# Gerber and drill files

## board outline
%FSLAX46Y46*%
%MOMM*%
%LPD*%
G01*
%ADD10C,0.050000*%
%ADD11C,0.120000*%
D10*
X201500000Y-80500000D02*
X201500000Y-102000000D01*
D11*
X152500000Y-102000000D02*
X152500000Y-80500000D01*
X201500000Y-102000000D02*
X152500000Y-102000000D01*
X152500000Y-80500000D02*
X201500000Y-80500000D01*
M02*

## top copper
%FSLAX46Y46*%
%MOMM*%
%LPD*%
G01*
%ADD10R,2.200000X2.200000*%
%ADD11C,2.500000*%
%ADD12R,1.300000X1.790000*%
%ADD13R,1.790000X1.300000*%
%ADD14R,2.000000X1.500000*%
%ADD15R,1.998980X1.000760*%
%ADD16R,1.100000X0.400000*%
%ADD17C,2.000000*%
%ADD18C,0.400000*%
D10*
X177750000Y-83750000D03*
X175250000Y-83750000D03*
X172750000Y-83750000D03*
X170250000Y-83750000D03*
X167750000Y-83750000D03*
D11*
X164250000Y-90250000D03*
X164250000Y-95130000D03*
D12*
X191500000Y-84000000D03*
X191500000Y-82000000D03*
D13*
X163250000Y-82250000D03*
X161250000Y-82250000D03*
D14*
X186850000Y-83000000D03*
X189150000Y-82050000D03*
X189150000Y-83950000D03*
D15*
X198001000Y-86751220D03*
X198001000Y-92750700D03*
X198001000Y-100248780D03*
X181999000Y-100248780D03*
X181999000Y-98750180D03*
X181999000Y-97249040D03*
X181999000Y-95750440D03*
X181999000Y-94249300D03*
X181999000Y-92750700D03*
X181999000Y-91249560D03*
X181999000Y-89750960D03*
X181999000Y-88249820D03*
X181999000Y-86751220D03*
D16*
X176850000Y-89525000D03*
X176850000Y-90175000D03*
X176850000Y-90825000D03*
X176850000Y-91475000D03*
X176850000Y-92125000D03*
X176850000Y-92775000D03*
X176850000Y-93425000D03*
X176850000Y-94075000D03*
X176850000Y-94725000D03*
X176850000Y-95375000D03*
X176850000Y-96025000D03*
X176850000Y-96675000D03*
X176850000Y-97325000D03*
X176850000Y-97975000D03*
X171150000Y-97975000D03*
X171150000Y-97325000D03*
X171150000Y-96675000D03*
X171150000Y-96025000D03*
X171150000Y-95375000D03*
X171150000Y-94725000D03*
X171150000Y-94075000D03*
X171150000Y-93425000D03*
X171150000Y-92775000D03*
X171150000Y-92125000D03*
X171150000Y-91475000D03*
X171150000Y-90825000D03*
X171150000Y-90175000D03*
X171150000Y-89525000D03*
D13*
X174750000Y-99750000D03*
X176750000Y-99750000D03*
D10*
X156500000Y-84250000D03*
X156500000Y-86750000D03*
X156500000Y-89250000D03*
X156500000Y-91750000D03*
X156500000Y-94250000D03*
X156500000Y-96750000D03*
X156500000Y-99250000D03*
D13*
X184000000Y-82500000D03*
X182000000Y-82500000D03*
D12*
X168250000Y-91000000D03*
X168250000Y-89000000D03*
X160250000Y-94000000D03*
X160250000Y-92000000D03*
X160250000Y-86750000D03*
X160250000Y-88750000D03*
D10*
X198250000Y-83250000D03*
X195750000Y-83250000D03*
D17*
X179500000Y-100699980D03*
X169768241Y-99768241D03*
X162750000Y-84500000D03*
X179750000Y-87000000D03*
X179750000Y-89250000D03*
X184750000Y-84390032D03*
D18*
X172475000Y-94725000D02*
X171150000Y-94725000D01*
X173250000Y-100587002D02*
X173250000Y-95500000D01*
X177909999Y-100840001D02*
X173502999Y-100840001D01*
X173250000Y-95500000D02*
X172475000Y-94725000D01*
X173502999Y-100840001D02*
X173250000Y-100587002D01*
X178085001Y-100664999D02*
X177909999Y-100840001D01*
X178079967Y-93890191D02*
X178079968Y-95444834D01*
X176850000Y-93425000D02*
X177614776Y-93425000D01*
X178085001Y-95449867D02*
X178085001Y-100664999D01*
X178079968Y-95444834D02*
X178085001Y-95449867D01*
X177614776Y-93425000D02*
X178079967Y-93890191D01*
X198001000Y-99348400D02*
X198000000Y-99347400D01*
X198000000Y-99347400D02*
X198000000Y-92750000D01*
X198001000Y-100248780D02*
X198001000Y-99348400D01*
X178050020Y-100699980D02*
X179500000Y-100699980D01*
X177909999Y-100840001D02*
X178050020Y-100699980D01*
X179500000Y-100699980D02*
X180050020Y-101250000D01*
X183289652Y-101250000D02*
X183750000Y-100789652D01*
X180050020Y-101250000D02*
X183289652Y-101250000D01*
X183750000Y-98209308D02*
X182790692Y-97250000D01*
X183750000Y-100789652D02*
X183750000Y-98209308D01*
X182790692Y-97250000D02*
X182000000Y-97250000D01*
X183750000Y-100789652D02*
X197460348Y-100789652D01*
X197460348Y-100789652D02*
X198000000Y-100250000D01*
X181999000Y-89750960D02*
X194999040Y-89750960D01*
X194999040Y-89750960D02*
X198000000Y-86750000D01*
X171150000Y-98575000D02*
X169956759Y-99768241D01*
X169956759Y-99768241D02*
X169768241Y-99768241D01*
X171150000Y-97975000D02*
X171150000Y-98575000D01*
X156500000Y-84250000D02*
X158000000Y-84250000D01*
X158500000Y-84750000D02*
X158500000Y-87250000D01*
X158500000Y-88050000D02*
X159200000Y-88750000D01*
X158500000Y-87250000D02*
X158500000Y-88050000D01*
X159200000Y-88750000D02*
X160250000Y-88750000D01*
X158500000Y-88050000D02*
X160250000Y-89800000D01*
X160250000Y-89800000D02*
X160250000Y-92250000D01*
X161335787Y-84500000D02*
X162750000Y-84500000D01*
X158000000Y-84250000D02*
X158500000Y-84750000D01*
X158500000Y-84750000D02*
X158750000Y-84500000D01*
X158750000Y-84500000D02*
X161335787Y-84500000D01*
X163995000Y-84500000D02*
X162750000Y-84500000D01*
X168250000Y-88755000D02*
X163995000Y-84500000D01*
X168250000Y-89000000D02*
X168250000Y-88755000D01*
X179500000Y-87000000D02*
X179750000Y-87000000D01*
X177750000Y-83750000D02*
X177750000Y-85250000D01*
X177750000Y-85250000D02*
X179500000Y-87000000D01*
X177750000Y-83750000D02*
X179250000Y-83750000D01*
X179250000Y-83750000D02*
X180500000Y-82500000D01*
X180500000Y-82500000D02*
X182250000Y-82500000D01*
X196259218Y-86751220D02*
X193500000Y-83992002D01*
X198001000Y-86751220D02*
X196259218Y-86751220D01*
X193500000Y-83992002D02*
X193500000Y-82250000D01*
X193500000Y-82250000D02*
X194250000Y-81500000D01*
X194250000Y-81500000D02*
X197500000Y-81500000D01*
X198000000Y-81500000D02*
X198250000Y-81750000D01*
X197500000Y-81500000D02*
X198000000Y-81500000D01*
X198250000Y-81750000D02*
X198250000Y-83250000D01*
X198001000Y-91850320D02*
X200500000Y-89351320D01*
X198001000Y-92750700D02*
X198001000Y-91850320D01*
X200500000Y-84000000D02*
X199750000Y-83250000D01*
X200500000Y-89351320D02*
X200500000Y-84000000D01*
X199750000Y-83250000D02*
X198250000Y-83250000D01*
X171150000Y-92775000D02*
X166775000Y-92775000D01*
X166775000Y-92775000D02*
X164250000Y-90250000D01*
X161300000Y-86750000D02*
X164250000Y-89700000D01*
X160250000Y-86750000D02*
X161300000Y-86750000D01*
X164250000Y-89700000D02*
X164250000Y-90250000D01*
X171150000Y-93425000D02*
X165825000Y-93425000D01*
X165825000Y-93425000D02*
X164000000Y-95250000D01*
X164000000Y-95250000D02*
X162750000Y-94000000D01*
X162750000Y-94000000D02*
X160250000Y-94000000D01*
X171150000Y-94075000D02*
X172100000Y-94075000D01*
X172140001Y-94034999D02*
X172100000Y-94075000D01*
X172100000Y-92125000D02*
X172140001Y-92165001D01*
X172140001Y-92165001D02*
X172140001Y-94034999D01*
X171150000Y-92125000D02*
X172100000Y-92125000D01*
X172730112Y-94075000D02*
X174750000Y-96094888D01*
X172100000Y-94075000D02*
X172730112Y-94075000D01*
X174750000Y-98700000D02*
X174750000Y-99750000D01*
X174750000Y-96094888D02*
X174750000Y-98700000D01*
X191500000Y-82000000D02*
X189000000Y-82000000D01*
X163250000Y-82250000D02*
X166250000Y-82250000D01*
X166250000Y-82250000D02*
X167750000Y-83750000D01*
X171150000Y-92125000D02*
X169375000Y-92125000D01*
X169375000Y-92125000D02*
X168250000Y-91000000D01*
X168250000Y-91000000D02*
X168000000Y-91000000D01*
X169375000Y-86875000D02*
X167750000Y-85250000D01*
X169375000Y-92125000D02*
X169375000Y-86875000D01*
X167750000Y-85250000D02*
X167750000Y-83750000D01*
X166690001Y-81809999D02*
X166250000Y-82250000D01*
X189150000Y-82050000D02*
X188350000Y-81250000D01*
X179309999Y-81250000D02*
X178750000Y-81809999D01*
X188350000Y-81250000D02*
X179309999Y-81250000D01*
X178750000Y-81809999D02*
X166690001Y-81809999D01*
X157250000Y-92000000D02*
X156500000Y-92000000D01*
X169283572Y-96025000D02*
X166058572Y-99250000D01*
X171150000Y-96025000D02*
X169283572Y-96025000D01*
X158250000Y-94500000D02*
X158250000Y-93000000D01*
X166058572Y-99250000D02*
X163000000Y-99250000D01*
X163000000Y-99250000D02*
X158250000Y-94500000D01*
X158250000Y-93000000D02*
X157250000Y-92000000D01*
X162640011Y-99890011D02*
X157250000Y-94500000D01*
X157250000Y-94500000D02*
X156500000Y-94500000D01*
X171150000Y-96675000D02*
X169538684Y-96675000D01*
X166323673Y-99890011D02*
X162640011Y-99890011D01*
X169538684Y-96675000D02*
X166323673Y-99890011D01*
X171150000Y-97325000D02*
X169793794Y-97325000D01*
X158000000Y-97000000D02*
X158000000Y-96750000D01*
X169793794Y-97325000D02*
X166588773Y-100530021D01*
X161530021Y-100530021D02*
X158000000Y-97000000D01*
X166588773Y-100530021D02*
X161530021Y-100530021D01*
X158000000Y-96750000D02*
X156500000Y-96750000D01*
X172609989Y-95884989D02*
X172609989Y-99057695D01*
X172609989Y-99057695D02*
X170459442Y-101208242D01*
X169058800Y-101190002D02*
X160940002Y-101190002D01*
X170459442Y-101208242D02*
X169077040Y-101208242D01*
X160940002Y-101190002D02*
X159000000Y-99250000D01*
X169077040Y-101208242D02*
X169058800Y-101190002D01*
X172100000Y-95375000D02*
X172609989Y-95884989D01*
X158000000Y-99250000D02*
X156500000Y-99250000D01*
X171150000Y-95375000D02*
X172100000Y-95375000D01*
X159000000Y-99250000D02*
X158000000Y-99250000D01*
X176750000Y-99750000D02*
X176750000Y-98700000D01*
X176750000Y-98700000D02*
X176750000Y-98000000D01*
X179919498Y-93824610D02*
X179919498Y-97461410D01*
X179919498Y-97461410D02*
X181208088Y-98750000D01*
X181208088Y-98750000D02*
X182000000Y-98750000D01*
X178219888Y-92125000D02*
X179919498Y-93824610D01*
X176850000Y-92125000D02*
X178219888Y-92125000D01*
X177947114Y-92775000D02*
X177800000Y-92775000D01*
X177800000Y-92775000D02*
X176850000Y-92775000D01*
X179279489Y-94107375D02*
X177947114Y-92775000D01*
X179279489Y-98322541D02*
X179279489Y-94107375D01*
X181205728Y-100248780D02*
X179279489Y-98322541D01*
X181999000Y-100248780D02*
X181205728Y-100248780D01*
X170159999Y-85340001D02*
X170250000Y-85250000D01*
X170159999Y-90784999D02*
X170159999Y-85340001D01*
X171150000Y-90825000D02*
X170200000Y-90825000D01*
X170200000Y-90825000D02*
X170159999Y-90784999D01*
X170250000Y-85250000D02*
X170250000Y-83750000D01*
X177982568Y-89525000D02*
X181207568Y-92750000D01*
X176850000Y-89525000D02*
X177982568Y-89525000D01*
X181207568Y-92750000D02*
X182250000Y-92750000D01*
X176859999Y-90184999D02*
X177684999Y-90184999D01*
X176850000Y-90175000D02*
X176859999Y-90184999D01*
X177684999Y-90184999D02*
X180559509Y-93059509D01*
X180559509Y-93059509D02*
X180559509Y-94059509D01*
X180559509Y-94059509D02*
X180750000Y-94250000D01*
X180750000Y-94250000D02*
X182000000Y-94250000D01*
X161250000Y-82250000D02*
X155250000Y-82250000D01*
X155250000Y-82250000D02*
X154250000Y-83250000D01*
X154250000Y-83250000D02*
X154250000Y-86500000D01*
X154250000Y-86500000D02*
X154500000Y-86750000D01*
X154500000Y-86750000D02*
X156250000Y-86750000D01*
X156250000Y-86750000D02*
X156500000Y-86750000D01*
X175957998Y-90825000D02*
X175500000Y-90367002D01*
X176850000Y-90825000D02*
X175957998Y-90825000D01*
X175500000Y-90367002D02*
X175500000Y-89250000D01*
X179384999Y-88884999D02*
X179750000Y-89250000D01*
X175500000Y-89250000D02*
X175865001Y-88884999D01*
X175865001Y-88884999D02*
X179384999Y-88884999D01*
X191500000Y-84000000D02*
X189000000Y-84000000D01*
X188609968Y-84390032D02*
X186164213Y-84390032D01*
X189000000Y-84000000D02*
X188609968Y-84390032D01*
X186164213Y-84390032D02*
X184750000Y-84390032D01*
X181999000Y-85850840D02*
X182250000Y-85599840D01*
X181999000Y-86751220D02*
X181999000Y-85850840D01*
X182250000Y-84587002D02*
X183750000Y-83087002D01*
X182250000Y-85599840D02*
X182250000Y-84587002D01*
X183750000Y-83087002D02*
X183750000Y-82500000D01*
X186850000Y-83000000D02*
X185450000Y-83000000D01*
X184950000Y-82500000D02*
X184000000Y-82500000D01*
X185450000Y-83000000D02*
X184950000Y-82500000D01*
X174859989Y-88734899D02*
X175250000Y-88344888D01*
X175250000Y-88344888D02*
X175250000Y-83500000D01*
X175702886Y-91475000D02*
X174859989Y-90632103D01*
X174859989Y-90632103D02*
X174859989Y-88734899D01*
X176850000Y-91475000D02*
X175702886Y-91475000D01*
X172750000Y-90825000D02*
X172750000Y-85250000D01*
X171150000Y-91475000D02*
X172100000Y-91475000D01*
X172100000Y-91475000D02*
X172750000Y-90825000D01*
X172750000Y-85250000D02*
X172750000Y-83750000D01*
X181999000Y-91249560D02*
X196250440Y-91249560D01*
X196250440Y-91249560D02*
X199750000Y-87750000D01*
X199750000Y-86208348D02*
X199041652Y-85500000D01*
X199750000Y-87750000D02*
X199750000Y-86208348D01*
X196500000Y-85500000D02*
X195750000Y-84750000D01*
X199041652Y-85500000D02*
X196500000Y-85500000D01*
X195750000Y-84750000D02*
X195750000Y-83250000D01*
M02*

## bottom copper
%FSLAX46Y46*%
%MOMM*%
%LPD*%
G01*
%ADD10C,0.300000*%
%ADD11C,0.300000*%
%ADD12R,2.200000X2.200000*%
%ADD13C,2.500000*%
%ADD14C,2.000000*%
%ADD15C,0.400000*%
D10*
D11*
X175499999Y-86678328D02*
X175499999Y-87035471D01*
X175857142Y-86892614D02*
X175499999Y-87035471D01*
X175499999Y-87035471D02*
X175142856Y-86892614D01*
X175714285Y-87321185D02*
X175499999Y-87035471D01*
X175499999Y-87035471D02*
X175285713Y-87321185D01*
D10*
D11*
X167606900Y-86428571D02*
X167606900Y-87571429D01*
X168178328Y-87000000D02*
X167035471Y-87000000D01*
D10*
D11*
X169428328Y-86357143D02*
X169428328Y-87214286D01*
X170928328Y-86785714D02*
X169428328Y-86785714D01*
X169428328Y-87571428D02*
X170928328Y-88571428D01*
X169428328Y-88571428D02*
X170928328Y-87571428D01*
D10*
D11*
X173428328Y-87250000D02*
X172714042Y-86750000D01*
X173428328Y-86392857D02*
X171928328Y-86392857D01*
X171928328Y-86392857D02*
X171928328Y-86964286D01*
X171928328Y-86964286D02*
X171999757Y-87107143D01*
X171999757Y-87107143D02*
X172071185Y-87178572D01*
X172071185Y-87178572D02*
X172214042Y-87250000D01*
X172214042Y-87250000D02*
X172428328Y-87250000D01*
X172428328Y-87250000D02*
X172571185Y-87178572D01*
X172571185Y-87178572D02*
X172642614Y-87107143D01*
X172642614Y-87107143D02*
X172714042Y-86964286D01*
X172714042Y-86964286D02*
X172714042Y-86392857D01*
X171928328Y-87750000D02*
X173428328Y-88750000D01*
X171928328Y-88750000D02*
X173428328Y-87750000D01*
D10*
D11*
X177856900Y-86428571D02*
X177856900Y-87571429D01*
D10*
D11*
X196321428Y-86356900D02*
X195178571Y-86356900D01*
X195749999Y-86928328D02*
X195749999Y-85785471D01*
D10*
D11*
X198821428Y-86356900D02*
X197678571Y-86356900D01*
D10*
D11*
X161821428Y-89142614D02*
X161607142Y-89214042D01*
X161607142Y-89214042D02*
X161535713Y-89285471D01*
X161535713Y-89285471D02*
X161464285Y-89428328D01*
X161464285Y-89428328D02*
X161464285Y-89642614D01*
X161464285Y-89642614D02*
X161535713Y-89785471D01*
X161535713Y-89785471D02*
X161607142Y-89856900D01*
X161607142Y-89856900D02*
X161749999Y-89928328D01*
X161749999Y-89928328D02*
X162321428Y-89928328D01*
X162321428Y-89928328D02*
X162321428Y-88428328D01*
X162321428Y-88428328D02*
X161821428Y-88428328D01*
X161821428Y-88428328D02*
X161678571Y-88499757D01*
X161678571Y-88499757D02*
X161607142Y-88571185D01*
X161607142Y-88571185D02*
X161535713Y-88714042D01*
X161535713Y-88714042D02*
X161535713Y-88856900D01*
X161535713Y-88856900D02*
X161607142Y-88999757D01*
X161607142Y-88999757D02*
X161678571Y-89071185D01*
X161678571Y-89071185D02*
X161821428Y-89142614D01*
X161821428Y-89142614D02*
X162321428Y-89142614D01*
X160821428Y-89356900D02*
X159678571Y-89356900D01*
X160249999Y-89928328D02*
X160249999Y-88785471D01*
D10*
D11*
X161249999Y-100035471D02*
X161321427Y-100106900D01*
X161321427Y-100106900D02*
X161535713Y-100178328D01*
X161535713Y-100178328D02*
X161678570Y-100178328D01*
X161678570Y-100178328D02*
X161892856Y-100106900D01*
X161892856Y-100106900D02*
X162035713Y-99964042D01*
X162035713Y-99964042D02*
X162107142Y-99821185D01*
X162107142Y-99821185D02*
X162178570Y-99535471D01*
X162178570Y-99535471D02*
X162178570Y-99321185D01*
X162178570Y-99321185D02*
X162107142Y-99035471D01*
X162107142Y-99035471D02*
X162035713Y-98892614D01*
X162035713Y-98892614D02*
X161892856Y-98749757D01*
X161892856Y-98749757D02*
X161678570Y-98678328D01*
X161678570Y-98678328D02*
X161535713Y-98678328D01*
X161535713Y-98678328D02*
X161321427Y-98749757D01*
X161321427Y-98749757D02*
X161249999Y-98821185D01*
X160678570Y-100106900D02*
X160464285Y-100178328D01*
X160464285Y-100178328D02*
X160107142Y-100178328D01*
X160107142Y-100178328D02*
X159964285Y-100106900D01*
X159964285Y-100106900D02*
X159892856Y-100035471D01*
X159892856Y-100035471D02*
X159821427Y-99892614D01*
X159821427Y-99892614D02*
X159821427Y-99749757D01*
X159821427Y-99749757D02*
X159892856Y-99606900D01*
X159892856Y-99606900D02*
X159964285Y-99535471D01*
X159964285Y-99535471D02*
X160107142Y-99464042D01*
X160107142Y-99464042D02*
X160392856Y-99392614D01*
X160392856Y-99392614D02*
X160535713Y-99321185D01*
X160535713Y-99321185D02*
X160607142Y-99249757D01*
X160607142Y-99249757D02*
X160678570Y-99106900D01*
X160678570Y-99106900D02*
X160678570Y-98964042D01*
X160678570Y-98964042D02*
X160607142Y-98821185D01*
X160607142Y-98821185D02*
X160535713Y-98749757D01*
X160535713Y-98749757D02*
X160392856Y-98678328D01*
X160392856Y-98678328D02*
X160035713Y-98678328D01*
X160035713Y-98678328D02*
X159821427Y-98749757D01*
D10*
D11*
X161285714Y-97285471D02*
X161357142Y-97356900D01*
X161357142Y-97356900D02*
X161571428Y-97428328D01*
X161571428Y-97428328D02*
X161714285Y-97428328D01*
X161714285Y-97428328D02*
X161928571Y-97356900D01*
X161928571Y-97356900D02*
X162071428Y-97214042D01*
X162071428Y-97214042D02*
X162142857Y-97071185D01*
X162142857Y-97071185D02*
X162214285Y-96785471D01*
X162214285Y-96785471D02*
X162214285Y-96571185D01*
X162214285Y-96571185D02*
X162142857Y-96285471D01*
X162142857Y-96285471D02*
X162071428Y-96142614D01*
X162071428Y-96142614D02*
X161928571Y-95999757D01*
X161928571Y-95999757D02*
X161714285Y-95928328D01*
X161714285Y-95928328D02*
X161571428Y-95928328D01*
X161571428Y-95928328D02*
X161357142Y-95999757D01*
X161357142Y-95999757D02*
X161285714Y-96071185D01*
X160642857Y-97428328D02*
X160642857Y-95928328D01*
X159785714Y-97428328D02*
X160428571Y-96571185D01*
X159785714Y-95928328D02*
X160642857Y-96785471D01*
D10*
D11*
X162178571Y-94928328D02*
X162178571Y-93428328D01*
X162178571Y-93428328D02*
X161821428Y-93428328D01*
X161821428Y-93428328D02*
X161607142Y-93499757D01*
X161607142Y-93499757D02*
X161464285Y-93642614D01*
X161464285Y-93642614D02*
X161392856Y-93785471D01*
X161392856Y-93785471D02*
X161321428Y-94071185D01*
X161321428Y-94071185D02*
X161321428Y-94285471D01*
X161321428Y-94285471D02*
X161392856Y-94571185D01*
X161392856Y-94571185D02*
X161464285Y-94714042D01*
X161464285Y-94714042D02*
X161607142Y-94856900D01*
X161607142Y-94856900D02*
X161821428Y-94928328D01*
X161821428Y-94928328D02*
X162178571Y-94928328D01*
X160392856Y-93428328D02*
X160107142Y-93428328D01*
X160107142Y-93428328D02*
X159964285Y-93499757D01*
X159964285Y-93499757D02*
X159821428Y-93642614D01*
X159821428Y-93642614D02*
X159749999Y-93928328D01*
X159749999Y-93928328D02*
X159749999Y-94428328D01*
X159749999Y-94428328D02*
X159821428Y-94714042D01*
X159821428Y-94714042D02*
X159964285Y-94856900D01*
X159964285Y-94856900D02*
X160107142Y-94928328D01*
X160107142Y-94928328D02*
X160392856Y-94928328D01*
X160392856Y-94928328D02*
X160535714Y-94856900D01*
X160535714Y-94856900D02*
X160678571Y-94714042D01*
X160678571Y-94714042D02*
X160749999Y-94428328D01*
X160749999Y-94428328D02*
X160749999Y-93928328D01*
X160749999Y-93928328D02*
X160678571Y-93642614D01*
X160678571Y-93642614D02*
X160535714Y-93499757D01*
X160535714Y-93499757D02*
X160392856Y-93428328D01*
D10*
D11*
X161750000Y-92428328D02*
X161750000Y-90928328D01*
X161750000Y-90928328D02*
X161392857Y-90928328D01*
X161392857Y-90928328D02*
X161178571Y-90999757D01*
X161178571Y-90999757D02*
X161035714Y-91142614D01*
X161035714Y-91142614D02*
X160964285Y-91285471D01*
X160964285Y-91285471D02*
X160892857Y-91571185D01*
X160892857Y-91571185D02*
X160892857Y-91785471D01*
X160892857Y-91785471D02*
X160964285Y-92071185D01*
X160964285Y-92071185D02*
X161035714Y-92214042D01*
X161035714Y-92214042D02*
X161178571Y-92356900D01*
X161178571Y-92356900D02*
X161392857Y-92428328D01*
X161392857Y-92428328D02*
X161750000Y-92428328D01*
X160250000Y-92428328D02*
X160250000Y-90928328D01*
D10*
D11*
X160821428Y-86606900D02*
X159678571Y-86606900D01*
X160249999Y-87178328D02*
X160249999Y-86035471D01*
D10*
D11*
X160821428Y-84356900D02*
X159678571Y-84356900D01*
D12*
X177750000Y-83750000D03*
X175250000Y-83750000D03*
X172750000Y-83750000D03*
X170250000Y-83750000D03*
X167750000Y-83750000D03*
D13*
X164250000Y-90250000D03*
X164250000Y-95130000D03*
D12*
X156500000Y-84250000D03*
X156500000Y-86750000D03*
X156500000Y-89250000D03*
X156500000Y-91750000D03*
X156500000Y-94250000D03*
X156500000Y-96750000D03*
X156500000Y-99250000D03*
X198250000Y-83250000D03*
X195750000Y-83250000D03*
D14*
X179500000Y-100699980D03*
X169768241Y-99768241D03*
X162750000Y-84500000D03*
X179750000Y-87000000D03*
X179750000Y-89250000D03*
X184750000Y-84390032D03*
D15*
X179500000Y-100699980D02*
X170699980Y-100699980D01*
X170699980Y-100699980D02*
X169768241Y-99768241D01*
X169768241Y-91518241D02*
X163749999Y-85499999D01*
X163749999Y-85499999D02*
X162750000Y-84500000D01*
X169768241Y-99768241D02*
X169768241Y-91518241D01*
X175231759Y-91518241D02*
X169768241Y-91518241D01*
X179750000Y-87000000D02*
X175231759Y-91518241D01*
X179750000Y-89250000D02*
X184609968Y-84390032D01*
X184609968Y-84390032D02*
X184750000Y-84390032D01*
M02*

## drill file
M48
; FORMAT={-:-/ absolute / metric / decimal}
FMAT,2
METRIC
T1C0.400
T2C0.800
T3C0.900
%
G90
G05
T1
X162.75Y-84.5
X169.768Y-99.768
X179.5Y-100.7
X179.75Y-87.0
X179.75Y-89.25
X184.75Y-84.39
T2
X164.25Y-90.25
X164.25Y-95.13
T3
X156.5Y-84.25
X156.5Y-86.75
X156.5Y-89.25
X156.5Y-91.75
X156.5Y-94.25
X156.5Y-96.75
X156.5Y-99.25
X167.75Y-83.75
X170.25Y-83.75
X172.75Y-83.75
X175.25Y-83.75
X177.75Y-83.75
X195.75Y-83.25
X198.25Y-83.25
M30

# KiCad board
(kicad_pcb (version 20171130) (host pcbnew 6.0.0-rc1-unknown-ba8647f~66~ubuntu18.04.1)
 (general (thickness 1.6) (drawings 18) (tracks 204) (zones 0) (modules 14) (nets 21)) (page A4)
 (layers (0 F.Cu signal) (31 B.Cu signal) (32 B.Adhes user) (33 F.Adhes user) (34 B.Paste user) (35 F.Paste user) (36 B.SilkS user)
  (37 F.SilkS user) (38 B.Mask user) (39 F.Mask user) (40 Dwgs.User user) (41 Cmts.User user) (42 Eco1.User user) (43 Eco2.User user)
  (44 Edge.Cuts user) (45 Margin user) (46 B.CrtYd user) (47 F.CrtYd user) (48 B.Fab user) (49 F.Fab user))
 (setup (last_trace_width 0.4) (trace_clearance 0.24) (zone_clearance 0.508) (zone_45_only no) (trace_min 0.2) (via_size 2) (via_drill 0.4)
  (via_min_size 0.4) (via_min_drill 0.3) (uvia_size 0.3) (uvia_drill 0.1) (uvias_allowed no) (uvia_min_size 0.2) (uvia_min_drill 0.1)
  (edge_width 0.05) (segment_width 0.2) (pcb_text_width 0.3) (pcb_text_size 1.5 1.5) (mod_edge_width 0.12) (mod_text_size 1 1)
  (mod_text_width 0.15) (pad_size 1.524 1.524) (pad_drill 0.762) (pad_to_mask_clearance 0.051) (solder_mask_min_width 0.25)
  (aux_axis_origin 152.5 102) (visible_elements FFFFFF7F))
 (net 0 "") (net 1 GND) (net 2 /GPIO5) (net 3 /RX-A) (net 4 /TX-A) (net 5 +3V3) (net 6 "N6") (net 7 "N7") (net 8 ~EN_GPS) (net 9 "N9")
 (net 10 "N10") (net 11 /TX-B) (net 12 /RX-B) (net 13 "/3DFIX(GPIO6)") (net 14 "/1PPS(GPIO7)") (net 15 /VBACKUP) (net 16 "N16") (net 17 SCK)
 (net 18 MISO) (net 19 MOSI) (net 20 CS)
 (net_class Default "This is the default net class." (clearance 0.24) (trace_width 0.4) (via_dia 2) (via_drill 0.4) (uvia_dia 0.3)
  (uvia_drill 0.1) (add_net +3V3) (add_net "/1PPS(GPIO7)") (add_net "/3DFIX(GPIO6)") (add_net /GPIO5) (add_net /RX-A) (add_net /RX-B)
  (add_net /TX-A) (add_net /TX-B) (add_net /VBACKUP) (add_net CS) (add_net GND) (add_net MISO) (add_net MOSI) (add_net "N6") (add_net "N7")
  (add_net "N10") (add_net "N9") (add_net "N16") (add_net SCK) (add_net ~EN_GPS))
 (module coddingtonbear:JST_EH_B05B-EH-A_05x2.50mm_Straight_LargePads (layer B.Cu) (at 167.75 83.75)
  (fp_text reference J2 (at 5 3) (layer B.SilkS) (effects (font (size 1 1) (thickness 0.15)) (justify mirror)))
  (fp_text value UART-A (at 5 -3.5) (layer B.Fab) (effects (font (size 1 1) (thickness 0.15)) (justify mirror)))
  (pad 5 thru_hole rect (at 10 0) (size 2.2 2.2) (drill 0.9) (layers *.Cu *.Mask) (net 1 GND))
  (pad 4 thru_hole rect (at 7.5 0) (size 2.2 2.2) (drill 0.9) (layers *.Cu *.Mask) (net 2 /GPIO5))
  (pad 3 thru_hole rect (at 5 0) (size 2.2 2.2) (drill 0.9) (layers *.Cu *.Mask) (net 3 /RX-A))
  (pad 2 thru_hole rect (at 2.5 0) (size 2.2 2.2) (drill 0.9) (layers *.Cu *.Mask) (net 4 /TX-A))
  (pad 1 thru_hole rect (at 0 0) (size 2.2 2.2) (drill 0.9) (layers *.Cu *.Mask) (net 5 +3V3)))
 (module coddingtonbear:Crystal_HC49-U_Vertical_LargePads (layer B.Cu) (at 164.25 90.25 270)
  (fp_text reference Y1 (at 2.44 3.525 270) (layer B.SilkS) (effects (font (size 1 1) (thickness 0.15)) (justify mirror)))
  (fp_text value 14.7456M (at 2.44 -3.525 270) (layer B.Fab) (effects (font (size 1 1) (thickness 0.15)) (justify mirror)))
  (pad 1 thru_hole circle (at 0 0 270) (size 2.5 2.5) (drill 0.8) (layers *.Cu *.Mask) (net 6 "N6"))
  (pad 2 thru_hole circle (at 4.88 0 270) (size 2.5 2.5) (drill 0.8) (layers *.Cu *.Mask) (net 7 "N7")))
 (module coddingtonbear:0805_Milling (layer F.Cu) (at 191.5 83 90)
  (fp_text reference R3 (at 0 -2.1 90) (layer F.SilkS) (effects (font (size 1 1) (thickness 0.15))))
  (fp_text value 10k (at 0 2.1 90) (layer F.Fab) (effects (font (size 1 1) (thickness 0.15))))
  (pad 1 smd rect (at -1 0 90) (size 1.79 1.3) (layers F.Cu F.Paste F.Mask) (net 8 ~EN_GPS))
  (pad 2 smd rect (at 1 0 90) (size 1.79 1.3) (layers F.Cu F.Paste F.Mask) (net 5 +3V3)))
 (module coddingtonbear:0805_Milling (layer F.Cu) (at 162.25 82.25 180)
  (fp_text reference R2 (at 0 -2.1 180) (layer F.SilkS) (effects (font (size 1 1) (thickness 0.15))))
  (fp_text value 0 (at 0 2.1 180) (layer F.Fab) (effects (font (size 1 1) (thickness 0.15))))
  (pad 1 smd rect (at -1 0 180) (size 1.79 1.3) (layers F.Cu F.Paste F.Mask) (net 5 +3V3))
  (pad 2 smd rect (at 1 0 180) (size 1.79 1.3) (layers F.Cu F.Paste F.Mask) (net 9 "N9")))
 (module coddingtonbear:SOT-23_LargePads (layer F.Cu) (at 188 83 180)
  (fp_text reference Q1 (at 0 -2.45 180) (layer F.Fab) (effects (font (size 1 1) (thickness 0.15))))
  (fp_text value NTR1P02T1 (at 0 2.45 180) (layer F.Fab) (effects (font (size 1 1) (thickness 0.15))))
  (pad 3 smd rect (at 1.15 0 180) (size 2 1.5) (layers F.Cu F.Paste F.Mask) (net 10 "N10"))
  (pad 2 smd rect (at -1.15 0.95 180) (size 2 1.5) (layers F.Cu F.Paste F.Mask) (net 5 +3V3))
  (pad 1 smd rect (at -1.15 -0.95 180) (size 2 1.5) (layers F.Cu F.Paste F.Mask) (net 8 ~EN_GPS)))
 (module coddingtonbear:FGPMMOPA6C (layer F.Cu) (at 190 93.5)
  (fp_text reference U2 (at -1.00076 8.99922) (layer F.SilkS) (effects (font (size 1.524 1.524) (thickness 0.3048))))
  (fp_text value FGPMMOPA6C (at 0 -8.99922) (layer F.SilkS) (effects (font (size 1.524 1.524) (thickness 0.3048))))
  (pad 13 smd rect (at 8.001 -6.74878) (size 1.99898 1.00076) (layers F.Cu F.Paste F.Mask) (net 1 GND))
  (pad 12 smd rect (at 8.001 -0.7493) (size 1.99898 1.00076) (layers F.Cu F.Paste F.Mask) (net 1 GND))
  (pad 11 smd rect (at 8.001 6.74878) (size 1.99898 1.00076) (layers F.Cu F.Paste F.Mask) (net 1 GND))
  (pad 10 smd rect (at -8.001 6.74878) (size 1.99898 1.00076) (layers F.Cu F.Paste F.Mask) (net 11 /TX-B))
  (pad 9 smd rect (at -8.001 5.25018) (size 1.99898 1.00076) (layers F.Cu F.Paste F.Mask) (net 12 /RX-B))
  (pad 8 smd rect (at -8.001 3.74904) (size 1.99898 1.00076) (layers F.Cu F.Paste F.Mask) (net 1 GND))
  (pad 7 smd rect (at -8.001 2.25044) (size 1.99898 1.00076) (layers F.Cu F.Paste F.Mask))
  (pad 6 smd rect (at -8.001 0.7493) (size 1.99898 1.00076) (layers F.Cu F.Paste F.Mask) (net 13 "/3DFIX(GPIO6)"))
  (pad 5 smd rect (at -8.001 -0.7493) (size 1.99898 1.00076) (layers F.Cu F.Paste F.Mask) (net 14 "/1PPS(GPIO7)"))
  (pad 4 smd rect (at -8.001 -2.25044) (size 1.99898 1.00076) (layers F.Cu F.Paste F.Mask) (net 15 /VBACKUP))
  (pad 3 smd rect (at -8.001 -3.74904) (size 1.99898 1.00076) (layers F.Cu F.Paste F.Mask) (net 1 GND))
  (pad 2 smd rect (at -8.001 -5.25018) (size 1.99898 1.00076) (layers F.Cu F.Paste F.Mask))
  (pad 1 smd rect (at -8.001 -6.74878) (size 1.99898 1.00076) (layers F.Cu F.Paste F.Mask) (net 10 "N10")))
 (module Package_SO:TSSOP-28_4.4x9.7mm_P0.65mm (layer F.Cu) (at 174 93.75)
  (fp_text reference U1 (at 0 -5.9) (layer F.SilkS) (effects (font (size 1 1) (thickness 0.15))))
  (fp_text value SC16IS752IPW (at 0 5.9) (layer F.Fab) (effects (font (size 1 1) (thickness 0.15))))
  (pad 28 smd rect (at 2.85 -4.225) (size 1.1 0.4) (layers F.Cu F.Paste F.Mask) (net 14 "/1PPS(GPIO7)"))
  (pad 27 smd rect (at 2.85 -3.575) (size 1.1 0.4) (layers F.Cu F.Paste F.Mask) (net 13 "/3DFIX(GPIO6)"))
  (pad 26 smd rect (at 2.85 -2.925) (size 1.1 0.4) (layers F.Cu F.Paste F.Mask) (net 8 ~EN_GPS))
  (pad 25 smd rect (at 2.85 -2.275) (size 1.1 0.4) (layers F.Cu F.Paste F.Mask) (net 2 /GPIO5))
  (pad 24 smd rect (at 2.85 -1.625) (size 1.1 0.4) (layers F.Cu F.Paste F.Mask) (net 12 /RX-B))
  (pad 23 smd rect (at 2.85 -0.975) (size 1.1 0.4) (layers F.Cu F.Paste F.Mask) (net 11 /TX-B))
  (pad 22 smd rect (at 2.85 -0.325) (size 1.1 0.4) (layers F.Cu F.Paste F.Mask) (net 1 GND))
  (pad 21 smd rect (at 2.85 0.325) (size 1.1 0.4) (layers F.Cu F.Paste F.Mask))
  (pad 20 smd rect (at 2.85 0.975) (size 1.1 0.4) (layers F.Cu F.Paste F.Mask))
  (pad 19 smd rect (at 2.85 1.625) (size 1.1 0.4) (layers F.Cu F.Paste F.Mask))
  (pad 18 smd rect (at 2.85 2.275) (size 1.1 0.4) (layers F.Cu F.Paste F.Mask))
  (pad 17 smd rect (at 2.85 2.925) (size 1.1 0.4) (layers F.Cu F.Paste F.Mask))
  (pad 16 smd rect (at 2.85 3.575) (size 1.1 0.4) (layers F.Cu F.Paste F.Mask))
  (pad 15 smd rect (at 2.85 4.225) (size 1.1 0.4) (layers F.Cu F.Paste F.Mask) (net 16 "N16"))
  (pad 14 smd rect (at -2.85 4.225) (size 1.1 0.4) (layers F.Cu F.Paste F.Mask) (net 1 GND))
  (pad 13 smd rect (at -2.85 3.575) (size 1.1 0.4) (layers F.Cu F.Paste F.Mask) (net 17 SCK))
  (pad 12 smd rect (at -2.85 2.925) (size 1.1 0.4) (layers F.Cu F.Paste F.Mask) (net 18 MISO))
  (pad 11 smd rect (at -2.85 2.275) (size 1.1 0.4) (layers F.Cu F.Paste F.Mask) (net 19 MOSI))
  (pad 10 smd rect (at -2.85 1.625) (size 1.1 0.4) (layers F.Cu F.Paste F.Mask) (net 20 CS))
  (pad 9 smd rect (at -2.85 0.975) (size 1.1 0.4) (layers F.Cu F.Paste F.Mask) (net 1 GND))
  (pad 8 smd rect (at -2.85 0.325) (size 1.1 0.4) (layers F.Cu F.Paste F.Mask) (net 5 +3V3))
  (pad 7 smd rect (at -2.85 -0.325) (size 1.1 0.4) (layers F.Cu F.Paste F.Mask) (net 7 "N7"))
  (pad 6 smd rect (at -2.85 -0.975) (size 1.1 0.4) (layers F.Cu F.Paste F.Mask) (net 6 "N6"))
  (pad 5 smd rect (at -2.85 -1.625) (size 1.1 0.4) (layers F.Cu F.Paste F.Mask) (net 5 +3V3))
  (pad 4 smd rect (at -2.85 -2.275) (size 1.1 0.4) (layers F.Cu F.Paste F.Mask) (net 3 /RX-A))
  (pad 3 smd rect (at -2.85 -2.925) (size 1.1 0.4) (layers F.Cu F.Paste F.Mask) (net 4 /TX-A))
  (pad 2 smd rect (at -2.85 -3.575) (size 1.1 0.4) (layers F.Cu F.Paste F.Mask))
  (pad 1 smd rect (at -2.85 -4.225) (size 1.1 0.4) (layers F.Cu F.Paste F.Mask)))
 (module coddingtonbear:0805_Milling (layer F.Cu) (at 175.75 99.75)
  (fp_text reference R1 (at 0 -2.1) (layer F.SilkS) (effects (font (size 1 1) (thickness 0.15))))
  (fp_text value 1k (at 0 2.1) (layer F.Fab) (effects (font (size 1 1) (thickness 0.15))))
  (pad 1 smd rect (at -1 0) (size 1.79 1.3) (layers F.Cu F.Paste F.Mask) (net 5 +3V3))
  (pad 2 smd rect (at 1 0) (size 1.79 1.3) (layers F.Cu F.Paste F.Mask) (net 16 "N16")))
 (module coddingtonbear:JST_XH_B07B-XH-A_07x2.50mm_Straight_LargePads (layer B.Cu) (at 156.5 99.25 90)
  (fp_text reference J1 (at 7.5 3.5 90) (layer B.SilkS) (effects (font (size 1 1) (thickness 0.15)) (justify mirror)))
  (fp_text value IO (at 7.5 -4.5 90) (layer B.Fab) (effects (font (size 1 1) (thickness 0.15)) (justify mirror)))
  (pad 7 thru_hole rect (at 15 0 90) (size 2.2 2.2) (drill 0.9) (layers *.Cu *.Mask) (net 1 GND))
  (pad 6 thru_hole rect (at 12.5 0 90) (size 2.2 2.2) (drill 0.9) (layers *.Cu *.Mask) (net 9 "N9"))
  (pad 5 thru_hole rect (at 10 0 90) (size 2.2 2.2) (drill 0.9) (layers *.Cu *.Mask))
  (pad 4 thru_hole rect (at 7.5 0 90) (size 2.2 2.2) (drill 0.9) (layers *.Cu *.Mask) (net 19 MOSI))
  (pad 3 thru_hole rect (at 5 0 90) (size 2.2 2.2) (drill 0.9) (layers *.Cu *.Mask) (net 18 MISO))
  (pad 2 thru_hole rect (at 2.5 0 90) (size 2.2 2.2) (drill 0.9) (layers *.Cu *.Mask) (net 17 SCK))
  (pad 1 thru_hole rect (at 0 0 90) (size 2.2 2.2) (drill 0.9) (layers *.Cu *.Mask) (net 20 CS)))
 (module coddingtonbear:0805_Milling (layer F.Cu) (at 183 82.5 180)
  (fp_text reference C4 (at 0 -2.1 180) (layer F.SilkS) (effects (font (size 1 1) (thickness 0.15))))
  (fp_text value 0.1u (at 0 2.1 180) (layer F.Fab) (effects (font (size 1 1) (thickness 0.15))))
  (pad 1 smd rect (at -1 0 180) (size 1.79 1.3) (layers F.Cu F.Paste F.Mask) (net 10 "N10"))
  (pad 2 smd rect (at 1 0 180) (size 1.79 1.3) (layers F.Cu F.Paste F.Mask) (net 1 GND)))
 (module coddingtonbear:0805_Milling (layer F.Cu) (at 168.25 90 90)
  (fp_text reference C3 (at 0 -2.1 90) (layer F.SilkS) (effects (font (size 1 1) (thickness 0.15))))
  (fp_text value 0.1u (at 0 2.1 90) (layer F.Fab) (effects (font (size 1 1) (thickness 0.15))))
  (pad 1 smd rect (at -1 0 90) (size 1.79 1.3) (layers F.Cu F.Paste F.Mask) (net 5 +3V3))
  (pad 2 smd rect (at 1 0 90) (size 1.79 1.3) (layers F.Cu F.Paste F.Mask) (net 1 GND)))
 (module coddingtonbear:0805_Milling (layer F.Cu) (at 160.25 93 90)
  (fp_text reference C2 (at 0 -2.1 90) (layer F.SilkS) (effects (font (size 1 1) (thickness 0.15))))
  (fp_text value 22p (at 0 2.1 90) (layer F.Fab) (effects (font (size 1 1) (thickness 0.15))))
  (pad 1 smd rect (at -1 0 90) (size 1.79 1.3) (layers F.Cu F.Paste F.Mask) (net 7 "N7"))
  (pad 2 smd rect (at 1 0 90) (size 1.79 1.3) (layers F.Cu F.Paste F.Mask) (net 1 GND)))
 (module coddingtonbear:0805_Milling (layer F.Cu) (at 160.25 87.75 270)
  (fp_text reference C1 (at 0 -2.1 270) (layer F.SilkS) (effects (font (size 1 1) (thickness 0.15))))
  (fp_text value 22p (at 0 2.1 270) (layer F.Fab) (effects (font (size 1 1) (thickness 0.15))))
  (pad 1 smd rect (at -1 0 270) (size 1.79 1.3) (layers F.Cu F.Paste F.Mask) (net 6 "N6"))
  (pad 2 smd rect (at 1 0 270) (size 1.79 1.3) (layers F.Cu F.Paste F.Mask) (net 1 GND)))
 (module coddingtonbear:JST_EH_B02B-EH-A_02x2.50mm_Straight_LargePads (layer B.Cu) (at 195.75 83.25)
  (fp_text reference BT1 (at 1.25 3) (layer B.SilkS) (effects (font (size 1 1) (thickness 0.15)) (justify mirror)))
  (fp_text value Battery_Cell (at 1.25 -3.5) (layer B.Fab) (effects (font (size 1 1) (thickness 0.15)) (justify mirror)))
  (pad 2 thru_hole rect (at 2.5 0) (size 2.2 2.2) (drill 0.9) (layers *.Cu *.Mask) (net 1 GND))
  (pad 1 thru_hole rect (at 0 0) (size 2.2 2.2) (drill 0.9) (layers *.Cu *.Mask) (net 15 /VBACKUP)))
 (gr_line (start 201.5 80.5) (end 201.5 102) (layer Edge.Cuts) (width 0.05))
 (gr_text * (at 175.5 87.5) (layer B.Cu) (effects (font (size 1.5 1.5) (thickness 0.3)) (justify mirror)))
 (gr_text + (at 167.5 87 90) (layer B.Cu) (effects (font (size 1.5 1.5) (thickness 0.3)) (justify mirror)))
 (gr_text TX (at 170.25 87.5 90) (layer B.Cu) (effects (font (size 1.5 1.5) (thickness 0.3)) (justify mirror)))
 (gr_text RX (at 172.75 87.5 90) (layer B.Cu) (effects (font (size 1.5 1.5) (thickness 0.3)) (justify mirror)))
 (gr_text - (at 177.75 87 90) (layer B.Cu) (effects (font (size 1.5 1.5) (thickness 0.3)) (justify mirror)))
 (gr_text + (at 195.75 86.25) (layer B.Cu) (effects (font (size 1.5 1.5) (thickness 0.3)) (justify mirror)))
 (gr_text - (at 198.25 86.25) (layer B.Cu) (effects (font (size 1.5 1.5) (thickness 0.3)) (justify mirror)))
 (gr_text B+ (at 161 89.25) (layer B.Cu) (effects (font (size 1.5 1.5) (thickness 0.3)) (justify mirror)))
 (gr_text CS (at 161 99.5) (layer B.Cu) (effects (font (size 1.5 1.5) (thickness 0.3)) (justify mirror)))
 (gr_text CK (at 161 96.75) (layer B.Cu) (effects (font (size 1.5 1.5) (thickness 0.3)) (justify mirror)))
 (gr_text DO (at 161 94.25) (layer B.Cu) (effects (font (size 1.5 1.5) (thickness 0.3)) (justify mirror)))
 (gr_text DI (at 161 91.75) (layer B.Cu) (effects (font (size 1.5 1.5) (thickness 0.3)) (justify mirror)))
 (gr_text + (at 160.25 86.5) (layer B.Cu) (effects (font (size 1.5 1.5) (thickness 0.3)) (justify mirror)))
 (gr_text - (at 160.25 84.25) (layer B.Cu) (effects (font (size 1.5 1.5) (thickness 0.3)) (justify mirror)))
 (gr_line (start 152.5 102) (end 152.5 80.5) (layer Edge.Cuts) (width 0.12))
 (gr_line (start 201.5 102) (end 152.5 102) (layer Edge.Cuts) (width 0.12))
 (gr_line (start 152.5 80.5) (end 201.5 80.5) (layer Edge.Cuts) (width 0.12))
 (segment (start 172.475 94.725) (end 171.15 94.725) (width 0.4) (layer F.Cu) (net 1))
 (segment (start 173.25 100.587002) (end 173.25 95.5) (width 0.4) (layer F.Cu) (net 1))
 (segment (start 177.909999 100.840001) (end 173.502999 100.840001) (width 0.4) (layer F.Cu) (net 1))
 (segment (start 173.25 95.5) (end 172.475 94.725) (width 0.4) (layer F.Cu) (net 1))
 (segment (start 173.502999 100.840001) (end 173.25 100.587002) (width 0.4) (layer F.Cu) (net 1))
 (segment (start 178.085001 100.664999) (end 177.909999 100.840001) (width 0.4) (layer F.Cu) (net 1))
 (segment (start 178.079967 93.890191) (end 178.079968 95.444834) (width 0.4) (layer F.Cu) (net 1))
 (segment (start 176.85 93.425) (end 177.614776 93.425) (width 0.4) (layer F.Cu) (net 1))
 (segment (start 178.085001 95.449867) (end 178.085001 100.664999) (width 0.4) (layer F.Cu) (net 1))
 (segment (start 178.079968 95.444834) (end 178.085001 95.449867) (width 0.4) (layer F.Cu) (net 1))
 (segment (start 177.614776 93.425) (end 178.079967 93.890191) (width 0.4) (layer F.Cu) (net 1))
 (segment (start 198.001 99.3484) (end 198 99.3474) (width 0.4) (layer F.Cu) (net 1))
 (segment (start 198 99.3474) (end 198 92.75) (width 0.4) (layer F.Cu) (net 1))
 (segment (start 198.001 100.24878) (end 198.001 99.3484) (width 0.4) (layer F.Cu) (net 1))
 (via (at 179.5 100.69998) (size 2) (drill 0.4) (layers F.Cu B.Cu) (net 1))
 (segment (start 178.05002 100.69998) (end 179.5 100.69998) (width 0.4) (layer F.Cu) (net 1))
 (segment (start 177.909999 100.840001) (end 178.05002 100.69998) (width 0.4) (layer F.Cu) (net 1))
 (segment (start 179.5 100.69998) (end 180.05002 101.25) (width 0.4) (layer F.Cu) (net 1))
 (segment (start 183.289652 101.25) (end 183.75 100.789652) (width 0.4) (layer F.Cu) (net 1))
 (segment (start 180.05002 101.25) (end 183.289652 101.25) (width 0.4) (layer F.Cu) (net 1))
 (segment (start 183.75 98.209308) (end 182.790692 97.25) (width 0.4) (layer F.Cu) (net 1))
 (segment (start 183.75 100.789652) (end 183.75 98.209308) (width 0.4) (layer F.Cu) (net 1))
 (segment (start 182.790692 97.25) (end 182 97.25) (width 0.4) (layer F.Cu) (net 1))
 (segment (start 183.75 100.789652) (end 197.460348 100.789652) (width 0.4) (layer F.Cu) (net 1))
 (segment (start 197.460348 100.789652) (end 198 100.25) (width 0.4) (layer F.Cu) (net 1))
 (segment (start 181.999 89.75096) (end 194.99904 89.75096) (width 0.4) (layer F.Cu) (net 1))
 (segment (start 194.99904 89.75096) (end 198 86.75) (width 0.4) (layer F.Cu) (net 1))
 (segment (start 171.15 98.575) (end 169.956759 99.768241) (width 0.4) (layer F.Cu) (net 1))
 (via (at 169.768241 99.768241) (size 2) (drill 0.4) (layers F.Cu B.Cu) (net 1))
 (segment (start 169.956759 99.768241) (end 169.768241 99.768241) (width 0.4) (layer F.Cu) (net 1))
 (segment (start 171.15 97.975) (end 171.15 98.575) (width 0.4) (layer F.Cu) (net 1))
 (segment (start 179.5 100.69998) (end 170.69998 100.69998) (width 0.4) (layer B.Cu) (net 1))
 (segment (start 170.69998 100.69998) (end 169.768241 99.768241) (width 0.4) (layer B.Cu) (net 1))
 (segment (start 156.5 84.25) (end 158 84.25) (width 0.4) (layer F.Cu) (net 1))
 (segment (start 158.5 84.75) (end 158.5 87.25) (width 0.4) (layer F.Cu) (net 1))
 (segment (start 158.5 88.05) (end 159.2 88.75) (width 0.4) (layer F.Cu) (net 1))
 (segment (start 158.5 87.25) (end 158.5 88.05) (width 0.4) (layer F.Cu) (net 1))
 (segment (start 159.2 88.75) (end 160.25 88.75) (width 0.4) (layer F.Cu) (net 1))
 (segment (start 158.5 88.05) (end 160.25 89.8) (width 0.4) (layer F.Cu) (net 1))
 (segment (start 160.25 89.8) (end 160.25 92.25) (width 0.4) (layer F.Cu) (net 1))
 (segment (start 161.335787 84.5) (end 162.75 84.5) (width 0.4) (layer F.Cu) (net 1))
 (segment (start 169.768241 91.518241) (end 163.749999 85.499999) (width 0.4) (layer B.Cu) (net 1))
 (segment (start 158 84.25) (end 158.5 84.75) (width 0.4) (layer F.Cu) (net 1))
 (segment (start 163.749999 85.499999) (end 162.75 84.5) (width 0.4) (layer B.Cu) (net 1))
 (segment (start 169.768241 99.768241) (end 169.768241 91.518241) (width 0.4) (layer B.Cu) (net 1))
 (segment (start 158.5 84.75) (end 158.75 84.5) (width 0.4) (layer F.Cu) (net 1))
 (segment (start 158.75 84.5) (end 161.335787 84.5) (width 0.4) (layer F.Cu) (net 1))
 (via (at 162.75 84.5) (size 2) (drill 0.4) (layers F.Cu B.Cu) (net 1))
 (segment (start 163.995 84.5) (end 162.75 84.5) (width 0.4) (layer F.Cu) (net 1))
 (segment (start 168.25 88.755) (end 163.995 84.5) (width 0.4) (layer F.Cu) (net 1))
 (segment (start 168.25 89) (end 168.25 88.755) (width 0.4) (layer F.Cu) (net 1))
 (via (at 179.75 87) (size 2) (drill 0.4) (layers F.Cu B.Cu) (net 1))
 (segment (start 179.5 87) (end 179.75 87) (width 0.4) (layer F.Cu) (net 1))
 (segment (start 177.75 83.75) (end 177.75 85.25) (width 0.4) (layer F.Cu) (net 1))
 (segment (start 177.75 85.25) (end 179.5 87) (width 0.4) (layer F.Cu) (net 1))
 (segment (start 175.231759 91.518241) (end 169.768241 91.518241) (width 0.4) (layer B.Cu) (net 1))
 (segment (start 179.75 87) (end 175.231759 91.518241) (width 0.4) (layer B.Cu) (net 1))
 (segment (start 177.75 83.75) (end 179.25 83.75) (width 0.4) (layer F.Cu) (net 1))
 (segment (start 179.25 83.75) (end 180.5 82.5) (width 0.4) (layer F.Cu) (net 1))
 (segment (start 180.5 82.5) (end 182.25 82.5) (width 0.4) (layer F.Cu) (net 1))
 (segment (start 196.259218 86.75122) (end 193.5 83.992002) (width 0.4) (layer F.Cu) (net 1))
 (segment (start 198.001 86.75122) (end 196.259218 86.75122) (width 0.4) (layer F.Cu) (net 1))
 (segment (start 193.5 83.992002) (end 193.5 82.25) (width 0.4) (layer F.Cu) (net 1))
 (segment (start 193.5 82.25) (end 194.25 81.5) (width 0.4) (layer F.Cu) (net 1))
 (segment (start 194.25 81.5) (end 197.5 81.5) (width 0.4) (layer F.Cu) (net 1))
 (segment (start 198 81.5) (end 198.25 81.75) (width 0.4) (layer F.Cu) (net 1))
 (segment (start 197.5 81.5) (end 198 81.5) (width 0.4) (layer F.Cu) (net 1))
 (segment (start 198.25 81.75) (end 198.25 83.25) (width 0.4) (layer F.Cu) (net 1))
 (segment (start 198.001 91.85032) (end 200.5 89.35132) (width 0.4) (layer F.Cu) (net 1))
 (segment (start 198.001 92.7507) (end 198.001 91.85032) (width 0.4) (layer F.Cu) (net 1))
 (segment (start 200.5 84) (end 199.75 83.25) (width 0.4) (layer F.Cu) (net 1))
 (segment (start 200.5 89.35132) (end 200.5 84) (width 0.4) (layer F.Cu) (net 1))
 (segment (start 199.75 83.25) (end 198.25 83.25) (width 0.4) (layer F.Cu) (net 1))
 (segment (start 171.15 92.775) (end 166.775 92.775) (width 0.4) (layer F.Cu) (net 6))
 (segment (start 166.775 92.775) (end 164.25 90.25) (width 0.4) (layer F.Cu) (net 6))
 (segment (start 161.3 86.75) (end 164.25 89.7) (width 0.4) (layer F.Cu) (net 6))
 (segment (start 160.25 86.75) (end 161.3 86.75) (width 0.4) (layer F.Cu) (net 6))
 (segment (start 164.25 89.7) (end 164.25 90.25) (width 0.4) (layer F.Cu) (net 6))
 (segment (start 171.15 93.425) (end 165.825 93.425) (width 0.4) (layer F.Cu) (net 7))
 (segment (start 165.825 93.425) (end 164 95.25) (width 0.4) (layer F.Cu) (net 7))
 (segment (start 164 95.25) (end 162.75 94) (width 0.4) (layer F.Cu) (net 7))
 (segment (start 162.75 94) (end 160.25 94) (width 0.4) (layer F.Cu) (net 7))
 (segment (start 171.15 94.075) (end 172.1 94.075) (width 0.4) (layer F.Cu) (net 5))
 (segment (start 172.140001 94.034999) (end 172.1 94.075) (width 0.4) (layer F.Cu) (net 5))
 (segment (start 172.1 92.125) (end 172.140001 92.165001) (width 0.4) (layer F.Cu) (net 5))
 (segment (start 172.140001 92.165001) (end 172.140001 94.034999) (width 0.4) (layer F.Cu) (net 5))
 (segment (start 171.15 92.125) (end 172.1 92.125) (width 0.4) (layer F.Cu) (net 5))
 (segment (start 172.730112 94.075) (end 174.75 96.094888) (width 0.4) (layer F.Cu) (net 5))
 (segment (start 172.1 94.075) (end 172.730112 94.075) (width 0.4) (layer F.Cu) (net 5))
 (segment (start 174.75 98.7) (end 174.75 99.75) (width 0.4) (layer F.Cu) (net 5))
 (segment (start 174.75 96.094888) (end 174.75 98.7) (width 0.4) (layer F.Cu) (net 5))
 (segment (start 191.5 82) (end 189 82) (width 0.4) (layer F.Cu) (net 5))
 (segment (start 163.25 82.25) (end 166.25 82.25) (width 0.4) (layer F.Cu) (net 5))
 (segment (start 166.25 82.25) (end 167.75 83.75) (width 0.4) (layer F.Cu) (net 5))
 (segment (start 171.15 92.125) (end 169.375 92.125) (width 0.4) (layer F.Cu) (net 5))
 (segment (start 169.375 92.125) (end 168.25 91) (width 0.4) (layer F.Cu) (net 5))
 (segment (start 168.25 91) (end 168 91) (width 0.4) (layer F.Cu) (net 5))
 (segment (start 169.375 86.875) (end 167.75 85.25) (width 0.4) (layer F.Cu) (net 5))
 (segment (start 169.375 92.125) (end 169.375 86.875) (width 0.4) (layer F.Cu) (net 5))
 (segment (start 167.75 85.25) (end 167.75 83.75) (width 0.4) (layer F.Cu) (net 5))
 (segment (start 166.690001 81.809999) (end 166.25 82.25) (width 0.4) (layer F.Cu) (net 5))
 (segment (start 189.15 82.05) (end 188.35 81.25) (width 0.4) (layer F.Cu) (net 5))
 (segment (start 179.309999 81.25) (end 178.75 81.809999) (width 0.4) (layer F.Cu) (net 5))
 (segment (start 188.35 81.25) (end 179.309999 81.25) (width 0.4) (layer F.Cu) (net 5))
 (segment (start 178.75 81.809999) (end 166.690001 81.809999) (width 0.4) (layer F.Cu) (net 5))
 (segment (start 157.25 92) (end 156.5 92) (width 0.4) (layer F.Cu) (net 19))
 (segment (start 169.283572 96.025) (end 166.058572 99.25) (width 0.4) (layer F.Cu) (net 19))
 (segment (start 171.15 96.025) (end 169.283572 96.025) (width 0.4) (layer F.Cu) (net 19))
 (segment (start 158.25 94.5) (end 158.25 93) (width 0.4) (layer F.Cu) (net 19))
 (segment (start 166.058572 99.25) (end 163 99.25) (width 0.4) (layer F.Cu) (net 19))
 (segment (start 163 99.25) (end 158.25 94.5) (width 0.4) (layer F.Cu) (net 19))
 (segment (start 158.25 93) (end 157.25 92) (width 0.4) (layer F.Cu) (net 19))
 (segment (start 162.640011 99.890011) (end 157.25 94.5) (width 0.4) (layer F.Cu) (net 18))
 (segment (start 157.25 94.5) (end 156.5 94.5) (width 0.4) (layer F.Cu) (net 18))
 (segment (start 171.15 96.675) (end 169.538684 96.675) (width 0.4) (layer F.Cu) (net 18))
 (segment (start 166.323673 99.890011) (end 162.640011 99.890011) (width 0.4) (layer F.Cu) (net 18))
 (segment (start 169.538684 96.675) (end 166.323673 99.890011) (width 0.4) (layer F.Cu) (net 18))
 (segment (start 171.15 97.325) (end 169.793794 97.325) (width 0.4) (layer F.Cu) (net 17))
 (segment (start 158 97) (end 158 96.75) (width 0.4) (layer F.Cu) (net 17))
 (segment (start 169.793794 97.325) (end 166.588773 100.530021) (width 0.4) (layer F.Cu) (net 17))
 (segment (start 161.530021 100.530021) (end 158 97) (width 0.4) (layer F.Cu) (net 17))
 (segment (start 166.588773 100.530021) (end 161.530021 100.530021) (width 0.4) (layer F.Cu) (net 17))
 (segment (start 158 96.75) (end 156.5 96.75) (width 0.4) (layer F.Cu) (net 17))
 (segment (start 172.609989 95.884989) (end 172.609989 99.057695) (width 0.4) (layer F.Cu) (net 20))
 (segment (start 172.609989 99.057695) (end 170.459442 101.208242) (width 0.4) (layer F.Cu) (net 20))
 (segment (start 169.0588 101.190002) (end 160.940002 101.190002) (width 0.4) (layer F.Cu) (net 20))
 (segment (start 170.459442 101.208242) (end 169.07704 101.208242) (width 0.4) (layer F.Cu) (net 20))
 (segment (start 160.940002 101.190002) (end 159 99.25) (width 0.4) (layer F.Cu) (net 20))
 (segment (start 169.07704 101.208242) (end 169.0588 101.190002) (width 0.4) (layer F.Cu) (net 20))
 (segment (start 172.1 95.375) (end 172.609989 95.884989) (width 0.4) (layer F.Cu) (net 20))
 (segment (start 158 99.25) (end 156.5 99.25) (width 0.4) (layer F.Cu) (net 20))
 (segment (start 171.15 95.375) (end 172.1 95.375) (width 0.4) (layer F.Cu) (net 20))
 (segment (start 159 99.25) (end 158 99.25) (width 0.4) (layer F.Cu) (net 20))
 (segment (start 176.75 99.75) (end 176.75 98.7) (width 0.4) (layer F.Cu) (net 16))
 (segment (start 176.75 98.7) (end 176.75 98) (width 0.4) (layer F.Cu) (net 16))
 (segment (start 179.919498 93.82461) (end 179.919498 97.46141) (width 0.4) (layer F.Cu) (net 12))
 (segment (start 179.919498 97.46141) (end 181.208088 98.75) (width 0.4) (layer F.Cu) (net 12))
 (segment (start 181.208088 98.75) (end 182 98.75) (width 0.4) (layer F.Cu) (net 12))
 (segment (start 178.219888 92.125) (end 179.919498 93.82461) (width 0.4) (layer F.Cu) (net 12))
 (segment (start 176.85 92.125) (end 178.219888 92.125) (width 0.4) (layer F.Cu) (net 12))
 (segment (start 177.947114 92.775) (end 177.8 92.775) (width 0.4) (layer F.Cu) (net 11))
 (segment (start 177.8 92.775) (end 176.85 92.775) (width 0.4) (layer F.Cu) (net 11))
 (segment (start 179.279489 94.107375) (end 177.947114 92.775) (width 0.4) (layer F.Cu) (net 11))
 (segment (start 179.279489 98.322541) (end 179.279489 94.107375) (width 0.4) (layer F.Cu) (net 11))
 (segment (start 181.205728 100.24878) (end 179.279489 98.322541) (width 0.4) (layer F.Cu) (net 11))
 (segment (start 181.999 100.24878) (end 181.205728 100.24878) (width 0.4) (layer F.Cu) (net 11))
 (segment (start 170.159999 85.340001) (end 170.25 85.25) (width 0.4) (layer F.Cu) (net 4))
 (segment (start 170.159999 90.784999) (end 170.159999 85.340001) (width 0.4) (layer F.Cu) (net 4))
 (segment (start 171.15 90.825) (end 170.2 90.825) (width 0.4) (layer F.Cu) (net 4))
 (segment (start 170.2 90.825) (end 170.159999 90.784999) (width 0.4) (layer F.Cu) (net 4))
 (segment (start 170.25 85.25) (end 170.25 83.75) (width 0.4) (layer F.Cu) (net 4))
 (segment (start 177.982568 89.525) (end 181.207568 92.75) (width 0.4) (layer F.Cu) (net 14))
 (segment (start 176.85 89.525) (end 177.982568 89.525) (width 0.4) (layer F.Cu) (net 14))
 (segment (start 181.207568 92.75) (end 182.25 92.75) (width 0.4) (layer F.Cu) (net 14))
 (segment (start 176.859999 90.184999) (end 177.684999 90.184999) (width 0.4) (layer F.Cu) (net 13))
 (segment (start 176.85 90.175) (end 176.859999 90.184999) (width 0.4) (layer F.Cu) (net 13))
 (segment (start 177.684999 90.184999) (end 180.559509 93.059509) (width 0.4) (layer F.Cu) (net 13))
 (segment (start 180.559509 93.059509) (end 180.559509 94.059509) (width 0.4) (layer F.Cu) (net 13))
 (segment (start 180.559509 94.059509) (end 180.75 94.25) (width 0.4) (layer F.Cu) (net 13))
 (segment (start 180.75 94.25) (end 182 94.25) (width 0.4) (layer F.Cu) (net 13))
 (segment (start 161.25 82.25) (end 155.25 82.25) (width 0.4) (layer F.Cu) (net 9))
 (segment (start 155.25 82.25) (end 154.25 83.25) (width 0.4) (layer F.Cu) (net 9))
 (segment (start 154.25 83.25) (end 154.25 86.5) (width 0.4) (layer F.Cu) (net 9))
 (segment (start 154.25 86.5) (end 154.5 86.75) (width 0.4) (layer F.Cu) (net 9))
 (segment (start 154.5 86.75) (end 156.25 86.75) (width 0.4) (layer F.Cu) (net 9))
 (segment (start 156.25 86.75) (end 156.5 86.75) (width 0.4) (layer F.Cu) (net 9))
 (segment (start 175.957998 90.825) (end 175.5 90.367002) (width 0.4) (layer F.Cu) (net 8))
 (segment (start 176.85 90.825) (end 175.957998 90.825) (width 0.4) (layer F.Cu) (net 8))
 (segment (start 175.5 90.367002) (end 175.5 89.25) (width 0.4) (layer F.Cu) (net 8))
 (segment (start 179.384999 88.884999) (end 179.75 89.25) (width 0.4) (layer F.Cu) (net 8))
 (segment (start 175.5 89.25) (end 175.865001 88.884999) (width 0.4) (layer F.Cu) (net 8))
 (via (at 179.75 89.25) (size 2) (drill 0.4) (layers F.Cu B.Cu) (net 8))
 (segment (start 175.865001 88.884999) (end 179.384999 88.884999) (width 0.4) (layer F.Cu) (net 8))
 (segment (start 191.5 84) (end 189 84) (width 0.4) (layer F.Cu) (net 8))
 (segment (start 188.609968 84.390032) (end 186.164213 84.390032) (width 0.4) (layer F.Cu) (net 8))
 (segment (start 189 84) (end 188.609968 84.390032) (width 0.4) (layer F.Cu) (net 8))
 (segment (start 179.75 89.25) (end 184.609968 84.390032) (width 0.4) (layer B.Cu) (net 8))
 (segment (start 184.609968 84.390032) (end 184.75 84.390032) (width 0.4) (layer B.Cu) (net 8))
 (via (at 184.75 84.390032) (size 2) (drill 0.4) (layers F.Cu B.Cu) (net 8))
 (segment (start 186.164213 84.390032) (end 184.75 84.390032) (width 0.4) (layer F.Cu) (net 8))
 (segment (start 181.999 85.85084) (end 182.25 85.59984) (width 0.4) (layer F.Cu) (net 10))
 (segment (start 181.999 86.75122) (end 181.999 85.85084) (width 0.4) (layer F.Cu) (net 10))
 (segment (start 182.25 84.587002) (end 183.75 83.087002) (width 0.4) (layer F.Cu) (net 10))
 (segment (start 182.25 85.59984) (end 182.25 84.587002) (width 0.4) (layer F.Cu) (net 10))
 (segment (start 183.75 83.087002) (end 183.75 82.5) (width 0.4) (layer F.Cu) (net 10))
 (segment (start 186.85 83) (end 185.45 83) (width 0.4) (layer F.Cu) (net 10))
 (segment (start 184.95 82.5) (end 184 82.5) (width 0.4) (layer F.Cu) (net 10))
 (segment (start 185.45 83) (end 184.95 82.5) (width 0.4) (layer F.Cu) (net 10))
 (segment (start 174.859989 88.734899) (end 175.25 88.344888) (width 0.4) (layer F.Cu) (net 2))
 (segment (start 175.25 88.344888) (end 175.25 83.5) (width 0.4) (layer F.Cu) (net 2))
 (segment (start 175.702886 91.475) (end 174.859989 90.632103) (width 0.4) (layer F.Cu) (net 2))
 (segment (start 174.859989 90.632103) (end 174.859989 88.734899) (width 0.4) (layer F.Cu) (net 2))
 (segment (start 176.85 91.475) (end 175.702886 91.475) (width 0.4) (layer F.Cu) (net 2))
 (segment (start 172.75 90.825) (end 172.75 85.25) (width 0.4) (layer F.Cu) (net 3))
 (segment (start 171.15 91.475) (end 172.1 91.475) (width 0.4) (layer F.Cu) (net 3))
 (segment (start 172.1 91.475) (end 172.75 90.825) (width 0.4) (layer F.Cu) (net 3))
 (segment (start 172.75 85.25) (end 172.75 83.75) (width 0.4) (layer F.Cu) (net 3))
 (segment (start 181.999 91.24956) (end 196.25044 91.24956) (width 0.4) (layer F.Cu) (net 15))
 (segment (start 196.25044 91.24956) (end 199.75 87.75) (width 0.4) (layer F.Cu) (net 15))
 (segment (start 199.75 86.208348) (end 199.041652 85.5) (width 0.4) (layer F.Cu) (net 15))
 (segment (start 199.75 87.75) (end 199.75 86.208348) (width 0.4) (layer F.Cu) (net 15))
 (segment (start 196.5 85.5) (end 195.75 84.75) (width 0.4) (layer F.Cu) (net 15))
 (segment (start 199.041652 85.5) (end 196.5 85.5) (width 0.4) (layer F.Cu) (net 15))
 (segment (start 195.75 84.75) (end 195.75 83.25) (width 0.4) (layer F.Cu) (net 15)))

